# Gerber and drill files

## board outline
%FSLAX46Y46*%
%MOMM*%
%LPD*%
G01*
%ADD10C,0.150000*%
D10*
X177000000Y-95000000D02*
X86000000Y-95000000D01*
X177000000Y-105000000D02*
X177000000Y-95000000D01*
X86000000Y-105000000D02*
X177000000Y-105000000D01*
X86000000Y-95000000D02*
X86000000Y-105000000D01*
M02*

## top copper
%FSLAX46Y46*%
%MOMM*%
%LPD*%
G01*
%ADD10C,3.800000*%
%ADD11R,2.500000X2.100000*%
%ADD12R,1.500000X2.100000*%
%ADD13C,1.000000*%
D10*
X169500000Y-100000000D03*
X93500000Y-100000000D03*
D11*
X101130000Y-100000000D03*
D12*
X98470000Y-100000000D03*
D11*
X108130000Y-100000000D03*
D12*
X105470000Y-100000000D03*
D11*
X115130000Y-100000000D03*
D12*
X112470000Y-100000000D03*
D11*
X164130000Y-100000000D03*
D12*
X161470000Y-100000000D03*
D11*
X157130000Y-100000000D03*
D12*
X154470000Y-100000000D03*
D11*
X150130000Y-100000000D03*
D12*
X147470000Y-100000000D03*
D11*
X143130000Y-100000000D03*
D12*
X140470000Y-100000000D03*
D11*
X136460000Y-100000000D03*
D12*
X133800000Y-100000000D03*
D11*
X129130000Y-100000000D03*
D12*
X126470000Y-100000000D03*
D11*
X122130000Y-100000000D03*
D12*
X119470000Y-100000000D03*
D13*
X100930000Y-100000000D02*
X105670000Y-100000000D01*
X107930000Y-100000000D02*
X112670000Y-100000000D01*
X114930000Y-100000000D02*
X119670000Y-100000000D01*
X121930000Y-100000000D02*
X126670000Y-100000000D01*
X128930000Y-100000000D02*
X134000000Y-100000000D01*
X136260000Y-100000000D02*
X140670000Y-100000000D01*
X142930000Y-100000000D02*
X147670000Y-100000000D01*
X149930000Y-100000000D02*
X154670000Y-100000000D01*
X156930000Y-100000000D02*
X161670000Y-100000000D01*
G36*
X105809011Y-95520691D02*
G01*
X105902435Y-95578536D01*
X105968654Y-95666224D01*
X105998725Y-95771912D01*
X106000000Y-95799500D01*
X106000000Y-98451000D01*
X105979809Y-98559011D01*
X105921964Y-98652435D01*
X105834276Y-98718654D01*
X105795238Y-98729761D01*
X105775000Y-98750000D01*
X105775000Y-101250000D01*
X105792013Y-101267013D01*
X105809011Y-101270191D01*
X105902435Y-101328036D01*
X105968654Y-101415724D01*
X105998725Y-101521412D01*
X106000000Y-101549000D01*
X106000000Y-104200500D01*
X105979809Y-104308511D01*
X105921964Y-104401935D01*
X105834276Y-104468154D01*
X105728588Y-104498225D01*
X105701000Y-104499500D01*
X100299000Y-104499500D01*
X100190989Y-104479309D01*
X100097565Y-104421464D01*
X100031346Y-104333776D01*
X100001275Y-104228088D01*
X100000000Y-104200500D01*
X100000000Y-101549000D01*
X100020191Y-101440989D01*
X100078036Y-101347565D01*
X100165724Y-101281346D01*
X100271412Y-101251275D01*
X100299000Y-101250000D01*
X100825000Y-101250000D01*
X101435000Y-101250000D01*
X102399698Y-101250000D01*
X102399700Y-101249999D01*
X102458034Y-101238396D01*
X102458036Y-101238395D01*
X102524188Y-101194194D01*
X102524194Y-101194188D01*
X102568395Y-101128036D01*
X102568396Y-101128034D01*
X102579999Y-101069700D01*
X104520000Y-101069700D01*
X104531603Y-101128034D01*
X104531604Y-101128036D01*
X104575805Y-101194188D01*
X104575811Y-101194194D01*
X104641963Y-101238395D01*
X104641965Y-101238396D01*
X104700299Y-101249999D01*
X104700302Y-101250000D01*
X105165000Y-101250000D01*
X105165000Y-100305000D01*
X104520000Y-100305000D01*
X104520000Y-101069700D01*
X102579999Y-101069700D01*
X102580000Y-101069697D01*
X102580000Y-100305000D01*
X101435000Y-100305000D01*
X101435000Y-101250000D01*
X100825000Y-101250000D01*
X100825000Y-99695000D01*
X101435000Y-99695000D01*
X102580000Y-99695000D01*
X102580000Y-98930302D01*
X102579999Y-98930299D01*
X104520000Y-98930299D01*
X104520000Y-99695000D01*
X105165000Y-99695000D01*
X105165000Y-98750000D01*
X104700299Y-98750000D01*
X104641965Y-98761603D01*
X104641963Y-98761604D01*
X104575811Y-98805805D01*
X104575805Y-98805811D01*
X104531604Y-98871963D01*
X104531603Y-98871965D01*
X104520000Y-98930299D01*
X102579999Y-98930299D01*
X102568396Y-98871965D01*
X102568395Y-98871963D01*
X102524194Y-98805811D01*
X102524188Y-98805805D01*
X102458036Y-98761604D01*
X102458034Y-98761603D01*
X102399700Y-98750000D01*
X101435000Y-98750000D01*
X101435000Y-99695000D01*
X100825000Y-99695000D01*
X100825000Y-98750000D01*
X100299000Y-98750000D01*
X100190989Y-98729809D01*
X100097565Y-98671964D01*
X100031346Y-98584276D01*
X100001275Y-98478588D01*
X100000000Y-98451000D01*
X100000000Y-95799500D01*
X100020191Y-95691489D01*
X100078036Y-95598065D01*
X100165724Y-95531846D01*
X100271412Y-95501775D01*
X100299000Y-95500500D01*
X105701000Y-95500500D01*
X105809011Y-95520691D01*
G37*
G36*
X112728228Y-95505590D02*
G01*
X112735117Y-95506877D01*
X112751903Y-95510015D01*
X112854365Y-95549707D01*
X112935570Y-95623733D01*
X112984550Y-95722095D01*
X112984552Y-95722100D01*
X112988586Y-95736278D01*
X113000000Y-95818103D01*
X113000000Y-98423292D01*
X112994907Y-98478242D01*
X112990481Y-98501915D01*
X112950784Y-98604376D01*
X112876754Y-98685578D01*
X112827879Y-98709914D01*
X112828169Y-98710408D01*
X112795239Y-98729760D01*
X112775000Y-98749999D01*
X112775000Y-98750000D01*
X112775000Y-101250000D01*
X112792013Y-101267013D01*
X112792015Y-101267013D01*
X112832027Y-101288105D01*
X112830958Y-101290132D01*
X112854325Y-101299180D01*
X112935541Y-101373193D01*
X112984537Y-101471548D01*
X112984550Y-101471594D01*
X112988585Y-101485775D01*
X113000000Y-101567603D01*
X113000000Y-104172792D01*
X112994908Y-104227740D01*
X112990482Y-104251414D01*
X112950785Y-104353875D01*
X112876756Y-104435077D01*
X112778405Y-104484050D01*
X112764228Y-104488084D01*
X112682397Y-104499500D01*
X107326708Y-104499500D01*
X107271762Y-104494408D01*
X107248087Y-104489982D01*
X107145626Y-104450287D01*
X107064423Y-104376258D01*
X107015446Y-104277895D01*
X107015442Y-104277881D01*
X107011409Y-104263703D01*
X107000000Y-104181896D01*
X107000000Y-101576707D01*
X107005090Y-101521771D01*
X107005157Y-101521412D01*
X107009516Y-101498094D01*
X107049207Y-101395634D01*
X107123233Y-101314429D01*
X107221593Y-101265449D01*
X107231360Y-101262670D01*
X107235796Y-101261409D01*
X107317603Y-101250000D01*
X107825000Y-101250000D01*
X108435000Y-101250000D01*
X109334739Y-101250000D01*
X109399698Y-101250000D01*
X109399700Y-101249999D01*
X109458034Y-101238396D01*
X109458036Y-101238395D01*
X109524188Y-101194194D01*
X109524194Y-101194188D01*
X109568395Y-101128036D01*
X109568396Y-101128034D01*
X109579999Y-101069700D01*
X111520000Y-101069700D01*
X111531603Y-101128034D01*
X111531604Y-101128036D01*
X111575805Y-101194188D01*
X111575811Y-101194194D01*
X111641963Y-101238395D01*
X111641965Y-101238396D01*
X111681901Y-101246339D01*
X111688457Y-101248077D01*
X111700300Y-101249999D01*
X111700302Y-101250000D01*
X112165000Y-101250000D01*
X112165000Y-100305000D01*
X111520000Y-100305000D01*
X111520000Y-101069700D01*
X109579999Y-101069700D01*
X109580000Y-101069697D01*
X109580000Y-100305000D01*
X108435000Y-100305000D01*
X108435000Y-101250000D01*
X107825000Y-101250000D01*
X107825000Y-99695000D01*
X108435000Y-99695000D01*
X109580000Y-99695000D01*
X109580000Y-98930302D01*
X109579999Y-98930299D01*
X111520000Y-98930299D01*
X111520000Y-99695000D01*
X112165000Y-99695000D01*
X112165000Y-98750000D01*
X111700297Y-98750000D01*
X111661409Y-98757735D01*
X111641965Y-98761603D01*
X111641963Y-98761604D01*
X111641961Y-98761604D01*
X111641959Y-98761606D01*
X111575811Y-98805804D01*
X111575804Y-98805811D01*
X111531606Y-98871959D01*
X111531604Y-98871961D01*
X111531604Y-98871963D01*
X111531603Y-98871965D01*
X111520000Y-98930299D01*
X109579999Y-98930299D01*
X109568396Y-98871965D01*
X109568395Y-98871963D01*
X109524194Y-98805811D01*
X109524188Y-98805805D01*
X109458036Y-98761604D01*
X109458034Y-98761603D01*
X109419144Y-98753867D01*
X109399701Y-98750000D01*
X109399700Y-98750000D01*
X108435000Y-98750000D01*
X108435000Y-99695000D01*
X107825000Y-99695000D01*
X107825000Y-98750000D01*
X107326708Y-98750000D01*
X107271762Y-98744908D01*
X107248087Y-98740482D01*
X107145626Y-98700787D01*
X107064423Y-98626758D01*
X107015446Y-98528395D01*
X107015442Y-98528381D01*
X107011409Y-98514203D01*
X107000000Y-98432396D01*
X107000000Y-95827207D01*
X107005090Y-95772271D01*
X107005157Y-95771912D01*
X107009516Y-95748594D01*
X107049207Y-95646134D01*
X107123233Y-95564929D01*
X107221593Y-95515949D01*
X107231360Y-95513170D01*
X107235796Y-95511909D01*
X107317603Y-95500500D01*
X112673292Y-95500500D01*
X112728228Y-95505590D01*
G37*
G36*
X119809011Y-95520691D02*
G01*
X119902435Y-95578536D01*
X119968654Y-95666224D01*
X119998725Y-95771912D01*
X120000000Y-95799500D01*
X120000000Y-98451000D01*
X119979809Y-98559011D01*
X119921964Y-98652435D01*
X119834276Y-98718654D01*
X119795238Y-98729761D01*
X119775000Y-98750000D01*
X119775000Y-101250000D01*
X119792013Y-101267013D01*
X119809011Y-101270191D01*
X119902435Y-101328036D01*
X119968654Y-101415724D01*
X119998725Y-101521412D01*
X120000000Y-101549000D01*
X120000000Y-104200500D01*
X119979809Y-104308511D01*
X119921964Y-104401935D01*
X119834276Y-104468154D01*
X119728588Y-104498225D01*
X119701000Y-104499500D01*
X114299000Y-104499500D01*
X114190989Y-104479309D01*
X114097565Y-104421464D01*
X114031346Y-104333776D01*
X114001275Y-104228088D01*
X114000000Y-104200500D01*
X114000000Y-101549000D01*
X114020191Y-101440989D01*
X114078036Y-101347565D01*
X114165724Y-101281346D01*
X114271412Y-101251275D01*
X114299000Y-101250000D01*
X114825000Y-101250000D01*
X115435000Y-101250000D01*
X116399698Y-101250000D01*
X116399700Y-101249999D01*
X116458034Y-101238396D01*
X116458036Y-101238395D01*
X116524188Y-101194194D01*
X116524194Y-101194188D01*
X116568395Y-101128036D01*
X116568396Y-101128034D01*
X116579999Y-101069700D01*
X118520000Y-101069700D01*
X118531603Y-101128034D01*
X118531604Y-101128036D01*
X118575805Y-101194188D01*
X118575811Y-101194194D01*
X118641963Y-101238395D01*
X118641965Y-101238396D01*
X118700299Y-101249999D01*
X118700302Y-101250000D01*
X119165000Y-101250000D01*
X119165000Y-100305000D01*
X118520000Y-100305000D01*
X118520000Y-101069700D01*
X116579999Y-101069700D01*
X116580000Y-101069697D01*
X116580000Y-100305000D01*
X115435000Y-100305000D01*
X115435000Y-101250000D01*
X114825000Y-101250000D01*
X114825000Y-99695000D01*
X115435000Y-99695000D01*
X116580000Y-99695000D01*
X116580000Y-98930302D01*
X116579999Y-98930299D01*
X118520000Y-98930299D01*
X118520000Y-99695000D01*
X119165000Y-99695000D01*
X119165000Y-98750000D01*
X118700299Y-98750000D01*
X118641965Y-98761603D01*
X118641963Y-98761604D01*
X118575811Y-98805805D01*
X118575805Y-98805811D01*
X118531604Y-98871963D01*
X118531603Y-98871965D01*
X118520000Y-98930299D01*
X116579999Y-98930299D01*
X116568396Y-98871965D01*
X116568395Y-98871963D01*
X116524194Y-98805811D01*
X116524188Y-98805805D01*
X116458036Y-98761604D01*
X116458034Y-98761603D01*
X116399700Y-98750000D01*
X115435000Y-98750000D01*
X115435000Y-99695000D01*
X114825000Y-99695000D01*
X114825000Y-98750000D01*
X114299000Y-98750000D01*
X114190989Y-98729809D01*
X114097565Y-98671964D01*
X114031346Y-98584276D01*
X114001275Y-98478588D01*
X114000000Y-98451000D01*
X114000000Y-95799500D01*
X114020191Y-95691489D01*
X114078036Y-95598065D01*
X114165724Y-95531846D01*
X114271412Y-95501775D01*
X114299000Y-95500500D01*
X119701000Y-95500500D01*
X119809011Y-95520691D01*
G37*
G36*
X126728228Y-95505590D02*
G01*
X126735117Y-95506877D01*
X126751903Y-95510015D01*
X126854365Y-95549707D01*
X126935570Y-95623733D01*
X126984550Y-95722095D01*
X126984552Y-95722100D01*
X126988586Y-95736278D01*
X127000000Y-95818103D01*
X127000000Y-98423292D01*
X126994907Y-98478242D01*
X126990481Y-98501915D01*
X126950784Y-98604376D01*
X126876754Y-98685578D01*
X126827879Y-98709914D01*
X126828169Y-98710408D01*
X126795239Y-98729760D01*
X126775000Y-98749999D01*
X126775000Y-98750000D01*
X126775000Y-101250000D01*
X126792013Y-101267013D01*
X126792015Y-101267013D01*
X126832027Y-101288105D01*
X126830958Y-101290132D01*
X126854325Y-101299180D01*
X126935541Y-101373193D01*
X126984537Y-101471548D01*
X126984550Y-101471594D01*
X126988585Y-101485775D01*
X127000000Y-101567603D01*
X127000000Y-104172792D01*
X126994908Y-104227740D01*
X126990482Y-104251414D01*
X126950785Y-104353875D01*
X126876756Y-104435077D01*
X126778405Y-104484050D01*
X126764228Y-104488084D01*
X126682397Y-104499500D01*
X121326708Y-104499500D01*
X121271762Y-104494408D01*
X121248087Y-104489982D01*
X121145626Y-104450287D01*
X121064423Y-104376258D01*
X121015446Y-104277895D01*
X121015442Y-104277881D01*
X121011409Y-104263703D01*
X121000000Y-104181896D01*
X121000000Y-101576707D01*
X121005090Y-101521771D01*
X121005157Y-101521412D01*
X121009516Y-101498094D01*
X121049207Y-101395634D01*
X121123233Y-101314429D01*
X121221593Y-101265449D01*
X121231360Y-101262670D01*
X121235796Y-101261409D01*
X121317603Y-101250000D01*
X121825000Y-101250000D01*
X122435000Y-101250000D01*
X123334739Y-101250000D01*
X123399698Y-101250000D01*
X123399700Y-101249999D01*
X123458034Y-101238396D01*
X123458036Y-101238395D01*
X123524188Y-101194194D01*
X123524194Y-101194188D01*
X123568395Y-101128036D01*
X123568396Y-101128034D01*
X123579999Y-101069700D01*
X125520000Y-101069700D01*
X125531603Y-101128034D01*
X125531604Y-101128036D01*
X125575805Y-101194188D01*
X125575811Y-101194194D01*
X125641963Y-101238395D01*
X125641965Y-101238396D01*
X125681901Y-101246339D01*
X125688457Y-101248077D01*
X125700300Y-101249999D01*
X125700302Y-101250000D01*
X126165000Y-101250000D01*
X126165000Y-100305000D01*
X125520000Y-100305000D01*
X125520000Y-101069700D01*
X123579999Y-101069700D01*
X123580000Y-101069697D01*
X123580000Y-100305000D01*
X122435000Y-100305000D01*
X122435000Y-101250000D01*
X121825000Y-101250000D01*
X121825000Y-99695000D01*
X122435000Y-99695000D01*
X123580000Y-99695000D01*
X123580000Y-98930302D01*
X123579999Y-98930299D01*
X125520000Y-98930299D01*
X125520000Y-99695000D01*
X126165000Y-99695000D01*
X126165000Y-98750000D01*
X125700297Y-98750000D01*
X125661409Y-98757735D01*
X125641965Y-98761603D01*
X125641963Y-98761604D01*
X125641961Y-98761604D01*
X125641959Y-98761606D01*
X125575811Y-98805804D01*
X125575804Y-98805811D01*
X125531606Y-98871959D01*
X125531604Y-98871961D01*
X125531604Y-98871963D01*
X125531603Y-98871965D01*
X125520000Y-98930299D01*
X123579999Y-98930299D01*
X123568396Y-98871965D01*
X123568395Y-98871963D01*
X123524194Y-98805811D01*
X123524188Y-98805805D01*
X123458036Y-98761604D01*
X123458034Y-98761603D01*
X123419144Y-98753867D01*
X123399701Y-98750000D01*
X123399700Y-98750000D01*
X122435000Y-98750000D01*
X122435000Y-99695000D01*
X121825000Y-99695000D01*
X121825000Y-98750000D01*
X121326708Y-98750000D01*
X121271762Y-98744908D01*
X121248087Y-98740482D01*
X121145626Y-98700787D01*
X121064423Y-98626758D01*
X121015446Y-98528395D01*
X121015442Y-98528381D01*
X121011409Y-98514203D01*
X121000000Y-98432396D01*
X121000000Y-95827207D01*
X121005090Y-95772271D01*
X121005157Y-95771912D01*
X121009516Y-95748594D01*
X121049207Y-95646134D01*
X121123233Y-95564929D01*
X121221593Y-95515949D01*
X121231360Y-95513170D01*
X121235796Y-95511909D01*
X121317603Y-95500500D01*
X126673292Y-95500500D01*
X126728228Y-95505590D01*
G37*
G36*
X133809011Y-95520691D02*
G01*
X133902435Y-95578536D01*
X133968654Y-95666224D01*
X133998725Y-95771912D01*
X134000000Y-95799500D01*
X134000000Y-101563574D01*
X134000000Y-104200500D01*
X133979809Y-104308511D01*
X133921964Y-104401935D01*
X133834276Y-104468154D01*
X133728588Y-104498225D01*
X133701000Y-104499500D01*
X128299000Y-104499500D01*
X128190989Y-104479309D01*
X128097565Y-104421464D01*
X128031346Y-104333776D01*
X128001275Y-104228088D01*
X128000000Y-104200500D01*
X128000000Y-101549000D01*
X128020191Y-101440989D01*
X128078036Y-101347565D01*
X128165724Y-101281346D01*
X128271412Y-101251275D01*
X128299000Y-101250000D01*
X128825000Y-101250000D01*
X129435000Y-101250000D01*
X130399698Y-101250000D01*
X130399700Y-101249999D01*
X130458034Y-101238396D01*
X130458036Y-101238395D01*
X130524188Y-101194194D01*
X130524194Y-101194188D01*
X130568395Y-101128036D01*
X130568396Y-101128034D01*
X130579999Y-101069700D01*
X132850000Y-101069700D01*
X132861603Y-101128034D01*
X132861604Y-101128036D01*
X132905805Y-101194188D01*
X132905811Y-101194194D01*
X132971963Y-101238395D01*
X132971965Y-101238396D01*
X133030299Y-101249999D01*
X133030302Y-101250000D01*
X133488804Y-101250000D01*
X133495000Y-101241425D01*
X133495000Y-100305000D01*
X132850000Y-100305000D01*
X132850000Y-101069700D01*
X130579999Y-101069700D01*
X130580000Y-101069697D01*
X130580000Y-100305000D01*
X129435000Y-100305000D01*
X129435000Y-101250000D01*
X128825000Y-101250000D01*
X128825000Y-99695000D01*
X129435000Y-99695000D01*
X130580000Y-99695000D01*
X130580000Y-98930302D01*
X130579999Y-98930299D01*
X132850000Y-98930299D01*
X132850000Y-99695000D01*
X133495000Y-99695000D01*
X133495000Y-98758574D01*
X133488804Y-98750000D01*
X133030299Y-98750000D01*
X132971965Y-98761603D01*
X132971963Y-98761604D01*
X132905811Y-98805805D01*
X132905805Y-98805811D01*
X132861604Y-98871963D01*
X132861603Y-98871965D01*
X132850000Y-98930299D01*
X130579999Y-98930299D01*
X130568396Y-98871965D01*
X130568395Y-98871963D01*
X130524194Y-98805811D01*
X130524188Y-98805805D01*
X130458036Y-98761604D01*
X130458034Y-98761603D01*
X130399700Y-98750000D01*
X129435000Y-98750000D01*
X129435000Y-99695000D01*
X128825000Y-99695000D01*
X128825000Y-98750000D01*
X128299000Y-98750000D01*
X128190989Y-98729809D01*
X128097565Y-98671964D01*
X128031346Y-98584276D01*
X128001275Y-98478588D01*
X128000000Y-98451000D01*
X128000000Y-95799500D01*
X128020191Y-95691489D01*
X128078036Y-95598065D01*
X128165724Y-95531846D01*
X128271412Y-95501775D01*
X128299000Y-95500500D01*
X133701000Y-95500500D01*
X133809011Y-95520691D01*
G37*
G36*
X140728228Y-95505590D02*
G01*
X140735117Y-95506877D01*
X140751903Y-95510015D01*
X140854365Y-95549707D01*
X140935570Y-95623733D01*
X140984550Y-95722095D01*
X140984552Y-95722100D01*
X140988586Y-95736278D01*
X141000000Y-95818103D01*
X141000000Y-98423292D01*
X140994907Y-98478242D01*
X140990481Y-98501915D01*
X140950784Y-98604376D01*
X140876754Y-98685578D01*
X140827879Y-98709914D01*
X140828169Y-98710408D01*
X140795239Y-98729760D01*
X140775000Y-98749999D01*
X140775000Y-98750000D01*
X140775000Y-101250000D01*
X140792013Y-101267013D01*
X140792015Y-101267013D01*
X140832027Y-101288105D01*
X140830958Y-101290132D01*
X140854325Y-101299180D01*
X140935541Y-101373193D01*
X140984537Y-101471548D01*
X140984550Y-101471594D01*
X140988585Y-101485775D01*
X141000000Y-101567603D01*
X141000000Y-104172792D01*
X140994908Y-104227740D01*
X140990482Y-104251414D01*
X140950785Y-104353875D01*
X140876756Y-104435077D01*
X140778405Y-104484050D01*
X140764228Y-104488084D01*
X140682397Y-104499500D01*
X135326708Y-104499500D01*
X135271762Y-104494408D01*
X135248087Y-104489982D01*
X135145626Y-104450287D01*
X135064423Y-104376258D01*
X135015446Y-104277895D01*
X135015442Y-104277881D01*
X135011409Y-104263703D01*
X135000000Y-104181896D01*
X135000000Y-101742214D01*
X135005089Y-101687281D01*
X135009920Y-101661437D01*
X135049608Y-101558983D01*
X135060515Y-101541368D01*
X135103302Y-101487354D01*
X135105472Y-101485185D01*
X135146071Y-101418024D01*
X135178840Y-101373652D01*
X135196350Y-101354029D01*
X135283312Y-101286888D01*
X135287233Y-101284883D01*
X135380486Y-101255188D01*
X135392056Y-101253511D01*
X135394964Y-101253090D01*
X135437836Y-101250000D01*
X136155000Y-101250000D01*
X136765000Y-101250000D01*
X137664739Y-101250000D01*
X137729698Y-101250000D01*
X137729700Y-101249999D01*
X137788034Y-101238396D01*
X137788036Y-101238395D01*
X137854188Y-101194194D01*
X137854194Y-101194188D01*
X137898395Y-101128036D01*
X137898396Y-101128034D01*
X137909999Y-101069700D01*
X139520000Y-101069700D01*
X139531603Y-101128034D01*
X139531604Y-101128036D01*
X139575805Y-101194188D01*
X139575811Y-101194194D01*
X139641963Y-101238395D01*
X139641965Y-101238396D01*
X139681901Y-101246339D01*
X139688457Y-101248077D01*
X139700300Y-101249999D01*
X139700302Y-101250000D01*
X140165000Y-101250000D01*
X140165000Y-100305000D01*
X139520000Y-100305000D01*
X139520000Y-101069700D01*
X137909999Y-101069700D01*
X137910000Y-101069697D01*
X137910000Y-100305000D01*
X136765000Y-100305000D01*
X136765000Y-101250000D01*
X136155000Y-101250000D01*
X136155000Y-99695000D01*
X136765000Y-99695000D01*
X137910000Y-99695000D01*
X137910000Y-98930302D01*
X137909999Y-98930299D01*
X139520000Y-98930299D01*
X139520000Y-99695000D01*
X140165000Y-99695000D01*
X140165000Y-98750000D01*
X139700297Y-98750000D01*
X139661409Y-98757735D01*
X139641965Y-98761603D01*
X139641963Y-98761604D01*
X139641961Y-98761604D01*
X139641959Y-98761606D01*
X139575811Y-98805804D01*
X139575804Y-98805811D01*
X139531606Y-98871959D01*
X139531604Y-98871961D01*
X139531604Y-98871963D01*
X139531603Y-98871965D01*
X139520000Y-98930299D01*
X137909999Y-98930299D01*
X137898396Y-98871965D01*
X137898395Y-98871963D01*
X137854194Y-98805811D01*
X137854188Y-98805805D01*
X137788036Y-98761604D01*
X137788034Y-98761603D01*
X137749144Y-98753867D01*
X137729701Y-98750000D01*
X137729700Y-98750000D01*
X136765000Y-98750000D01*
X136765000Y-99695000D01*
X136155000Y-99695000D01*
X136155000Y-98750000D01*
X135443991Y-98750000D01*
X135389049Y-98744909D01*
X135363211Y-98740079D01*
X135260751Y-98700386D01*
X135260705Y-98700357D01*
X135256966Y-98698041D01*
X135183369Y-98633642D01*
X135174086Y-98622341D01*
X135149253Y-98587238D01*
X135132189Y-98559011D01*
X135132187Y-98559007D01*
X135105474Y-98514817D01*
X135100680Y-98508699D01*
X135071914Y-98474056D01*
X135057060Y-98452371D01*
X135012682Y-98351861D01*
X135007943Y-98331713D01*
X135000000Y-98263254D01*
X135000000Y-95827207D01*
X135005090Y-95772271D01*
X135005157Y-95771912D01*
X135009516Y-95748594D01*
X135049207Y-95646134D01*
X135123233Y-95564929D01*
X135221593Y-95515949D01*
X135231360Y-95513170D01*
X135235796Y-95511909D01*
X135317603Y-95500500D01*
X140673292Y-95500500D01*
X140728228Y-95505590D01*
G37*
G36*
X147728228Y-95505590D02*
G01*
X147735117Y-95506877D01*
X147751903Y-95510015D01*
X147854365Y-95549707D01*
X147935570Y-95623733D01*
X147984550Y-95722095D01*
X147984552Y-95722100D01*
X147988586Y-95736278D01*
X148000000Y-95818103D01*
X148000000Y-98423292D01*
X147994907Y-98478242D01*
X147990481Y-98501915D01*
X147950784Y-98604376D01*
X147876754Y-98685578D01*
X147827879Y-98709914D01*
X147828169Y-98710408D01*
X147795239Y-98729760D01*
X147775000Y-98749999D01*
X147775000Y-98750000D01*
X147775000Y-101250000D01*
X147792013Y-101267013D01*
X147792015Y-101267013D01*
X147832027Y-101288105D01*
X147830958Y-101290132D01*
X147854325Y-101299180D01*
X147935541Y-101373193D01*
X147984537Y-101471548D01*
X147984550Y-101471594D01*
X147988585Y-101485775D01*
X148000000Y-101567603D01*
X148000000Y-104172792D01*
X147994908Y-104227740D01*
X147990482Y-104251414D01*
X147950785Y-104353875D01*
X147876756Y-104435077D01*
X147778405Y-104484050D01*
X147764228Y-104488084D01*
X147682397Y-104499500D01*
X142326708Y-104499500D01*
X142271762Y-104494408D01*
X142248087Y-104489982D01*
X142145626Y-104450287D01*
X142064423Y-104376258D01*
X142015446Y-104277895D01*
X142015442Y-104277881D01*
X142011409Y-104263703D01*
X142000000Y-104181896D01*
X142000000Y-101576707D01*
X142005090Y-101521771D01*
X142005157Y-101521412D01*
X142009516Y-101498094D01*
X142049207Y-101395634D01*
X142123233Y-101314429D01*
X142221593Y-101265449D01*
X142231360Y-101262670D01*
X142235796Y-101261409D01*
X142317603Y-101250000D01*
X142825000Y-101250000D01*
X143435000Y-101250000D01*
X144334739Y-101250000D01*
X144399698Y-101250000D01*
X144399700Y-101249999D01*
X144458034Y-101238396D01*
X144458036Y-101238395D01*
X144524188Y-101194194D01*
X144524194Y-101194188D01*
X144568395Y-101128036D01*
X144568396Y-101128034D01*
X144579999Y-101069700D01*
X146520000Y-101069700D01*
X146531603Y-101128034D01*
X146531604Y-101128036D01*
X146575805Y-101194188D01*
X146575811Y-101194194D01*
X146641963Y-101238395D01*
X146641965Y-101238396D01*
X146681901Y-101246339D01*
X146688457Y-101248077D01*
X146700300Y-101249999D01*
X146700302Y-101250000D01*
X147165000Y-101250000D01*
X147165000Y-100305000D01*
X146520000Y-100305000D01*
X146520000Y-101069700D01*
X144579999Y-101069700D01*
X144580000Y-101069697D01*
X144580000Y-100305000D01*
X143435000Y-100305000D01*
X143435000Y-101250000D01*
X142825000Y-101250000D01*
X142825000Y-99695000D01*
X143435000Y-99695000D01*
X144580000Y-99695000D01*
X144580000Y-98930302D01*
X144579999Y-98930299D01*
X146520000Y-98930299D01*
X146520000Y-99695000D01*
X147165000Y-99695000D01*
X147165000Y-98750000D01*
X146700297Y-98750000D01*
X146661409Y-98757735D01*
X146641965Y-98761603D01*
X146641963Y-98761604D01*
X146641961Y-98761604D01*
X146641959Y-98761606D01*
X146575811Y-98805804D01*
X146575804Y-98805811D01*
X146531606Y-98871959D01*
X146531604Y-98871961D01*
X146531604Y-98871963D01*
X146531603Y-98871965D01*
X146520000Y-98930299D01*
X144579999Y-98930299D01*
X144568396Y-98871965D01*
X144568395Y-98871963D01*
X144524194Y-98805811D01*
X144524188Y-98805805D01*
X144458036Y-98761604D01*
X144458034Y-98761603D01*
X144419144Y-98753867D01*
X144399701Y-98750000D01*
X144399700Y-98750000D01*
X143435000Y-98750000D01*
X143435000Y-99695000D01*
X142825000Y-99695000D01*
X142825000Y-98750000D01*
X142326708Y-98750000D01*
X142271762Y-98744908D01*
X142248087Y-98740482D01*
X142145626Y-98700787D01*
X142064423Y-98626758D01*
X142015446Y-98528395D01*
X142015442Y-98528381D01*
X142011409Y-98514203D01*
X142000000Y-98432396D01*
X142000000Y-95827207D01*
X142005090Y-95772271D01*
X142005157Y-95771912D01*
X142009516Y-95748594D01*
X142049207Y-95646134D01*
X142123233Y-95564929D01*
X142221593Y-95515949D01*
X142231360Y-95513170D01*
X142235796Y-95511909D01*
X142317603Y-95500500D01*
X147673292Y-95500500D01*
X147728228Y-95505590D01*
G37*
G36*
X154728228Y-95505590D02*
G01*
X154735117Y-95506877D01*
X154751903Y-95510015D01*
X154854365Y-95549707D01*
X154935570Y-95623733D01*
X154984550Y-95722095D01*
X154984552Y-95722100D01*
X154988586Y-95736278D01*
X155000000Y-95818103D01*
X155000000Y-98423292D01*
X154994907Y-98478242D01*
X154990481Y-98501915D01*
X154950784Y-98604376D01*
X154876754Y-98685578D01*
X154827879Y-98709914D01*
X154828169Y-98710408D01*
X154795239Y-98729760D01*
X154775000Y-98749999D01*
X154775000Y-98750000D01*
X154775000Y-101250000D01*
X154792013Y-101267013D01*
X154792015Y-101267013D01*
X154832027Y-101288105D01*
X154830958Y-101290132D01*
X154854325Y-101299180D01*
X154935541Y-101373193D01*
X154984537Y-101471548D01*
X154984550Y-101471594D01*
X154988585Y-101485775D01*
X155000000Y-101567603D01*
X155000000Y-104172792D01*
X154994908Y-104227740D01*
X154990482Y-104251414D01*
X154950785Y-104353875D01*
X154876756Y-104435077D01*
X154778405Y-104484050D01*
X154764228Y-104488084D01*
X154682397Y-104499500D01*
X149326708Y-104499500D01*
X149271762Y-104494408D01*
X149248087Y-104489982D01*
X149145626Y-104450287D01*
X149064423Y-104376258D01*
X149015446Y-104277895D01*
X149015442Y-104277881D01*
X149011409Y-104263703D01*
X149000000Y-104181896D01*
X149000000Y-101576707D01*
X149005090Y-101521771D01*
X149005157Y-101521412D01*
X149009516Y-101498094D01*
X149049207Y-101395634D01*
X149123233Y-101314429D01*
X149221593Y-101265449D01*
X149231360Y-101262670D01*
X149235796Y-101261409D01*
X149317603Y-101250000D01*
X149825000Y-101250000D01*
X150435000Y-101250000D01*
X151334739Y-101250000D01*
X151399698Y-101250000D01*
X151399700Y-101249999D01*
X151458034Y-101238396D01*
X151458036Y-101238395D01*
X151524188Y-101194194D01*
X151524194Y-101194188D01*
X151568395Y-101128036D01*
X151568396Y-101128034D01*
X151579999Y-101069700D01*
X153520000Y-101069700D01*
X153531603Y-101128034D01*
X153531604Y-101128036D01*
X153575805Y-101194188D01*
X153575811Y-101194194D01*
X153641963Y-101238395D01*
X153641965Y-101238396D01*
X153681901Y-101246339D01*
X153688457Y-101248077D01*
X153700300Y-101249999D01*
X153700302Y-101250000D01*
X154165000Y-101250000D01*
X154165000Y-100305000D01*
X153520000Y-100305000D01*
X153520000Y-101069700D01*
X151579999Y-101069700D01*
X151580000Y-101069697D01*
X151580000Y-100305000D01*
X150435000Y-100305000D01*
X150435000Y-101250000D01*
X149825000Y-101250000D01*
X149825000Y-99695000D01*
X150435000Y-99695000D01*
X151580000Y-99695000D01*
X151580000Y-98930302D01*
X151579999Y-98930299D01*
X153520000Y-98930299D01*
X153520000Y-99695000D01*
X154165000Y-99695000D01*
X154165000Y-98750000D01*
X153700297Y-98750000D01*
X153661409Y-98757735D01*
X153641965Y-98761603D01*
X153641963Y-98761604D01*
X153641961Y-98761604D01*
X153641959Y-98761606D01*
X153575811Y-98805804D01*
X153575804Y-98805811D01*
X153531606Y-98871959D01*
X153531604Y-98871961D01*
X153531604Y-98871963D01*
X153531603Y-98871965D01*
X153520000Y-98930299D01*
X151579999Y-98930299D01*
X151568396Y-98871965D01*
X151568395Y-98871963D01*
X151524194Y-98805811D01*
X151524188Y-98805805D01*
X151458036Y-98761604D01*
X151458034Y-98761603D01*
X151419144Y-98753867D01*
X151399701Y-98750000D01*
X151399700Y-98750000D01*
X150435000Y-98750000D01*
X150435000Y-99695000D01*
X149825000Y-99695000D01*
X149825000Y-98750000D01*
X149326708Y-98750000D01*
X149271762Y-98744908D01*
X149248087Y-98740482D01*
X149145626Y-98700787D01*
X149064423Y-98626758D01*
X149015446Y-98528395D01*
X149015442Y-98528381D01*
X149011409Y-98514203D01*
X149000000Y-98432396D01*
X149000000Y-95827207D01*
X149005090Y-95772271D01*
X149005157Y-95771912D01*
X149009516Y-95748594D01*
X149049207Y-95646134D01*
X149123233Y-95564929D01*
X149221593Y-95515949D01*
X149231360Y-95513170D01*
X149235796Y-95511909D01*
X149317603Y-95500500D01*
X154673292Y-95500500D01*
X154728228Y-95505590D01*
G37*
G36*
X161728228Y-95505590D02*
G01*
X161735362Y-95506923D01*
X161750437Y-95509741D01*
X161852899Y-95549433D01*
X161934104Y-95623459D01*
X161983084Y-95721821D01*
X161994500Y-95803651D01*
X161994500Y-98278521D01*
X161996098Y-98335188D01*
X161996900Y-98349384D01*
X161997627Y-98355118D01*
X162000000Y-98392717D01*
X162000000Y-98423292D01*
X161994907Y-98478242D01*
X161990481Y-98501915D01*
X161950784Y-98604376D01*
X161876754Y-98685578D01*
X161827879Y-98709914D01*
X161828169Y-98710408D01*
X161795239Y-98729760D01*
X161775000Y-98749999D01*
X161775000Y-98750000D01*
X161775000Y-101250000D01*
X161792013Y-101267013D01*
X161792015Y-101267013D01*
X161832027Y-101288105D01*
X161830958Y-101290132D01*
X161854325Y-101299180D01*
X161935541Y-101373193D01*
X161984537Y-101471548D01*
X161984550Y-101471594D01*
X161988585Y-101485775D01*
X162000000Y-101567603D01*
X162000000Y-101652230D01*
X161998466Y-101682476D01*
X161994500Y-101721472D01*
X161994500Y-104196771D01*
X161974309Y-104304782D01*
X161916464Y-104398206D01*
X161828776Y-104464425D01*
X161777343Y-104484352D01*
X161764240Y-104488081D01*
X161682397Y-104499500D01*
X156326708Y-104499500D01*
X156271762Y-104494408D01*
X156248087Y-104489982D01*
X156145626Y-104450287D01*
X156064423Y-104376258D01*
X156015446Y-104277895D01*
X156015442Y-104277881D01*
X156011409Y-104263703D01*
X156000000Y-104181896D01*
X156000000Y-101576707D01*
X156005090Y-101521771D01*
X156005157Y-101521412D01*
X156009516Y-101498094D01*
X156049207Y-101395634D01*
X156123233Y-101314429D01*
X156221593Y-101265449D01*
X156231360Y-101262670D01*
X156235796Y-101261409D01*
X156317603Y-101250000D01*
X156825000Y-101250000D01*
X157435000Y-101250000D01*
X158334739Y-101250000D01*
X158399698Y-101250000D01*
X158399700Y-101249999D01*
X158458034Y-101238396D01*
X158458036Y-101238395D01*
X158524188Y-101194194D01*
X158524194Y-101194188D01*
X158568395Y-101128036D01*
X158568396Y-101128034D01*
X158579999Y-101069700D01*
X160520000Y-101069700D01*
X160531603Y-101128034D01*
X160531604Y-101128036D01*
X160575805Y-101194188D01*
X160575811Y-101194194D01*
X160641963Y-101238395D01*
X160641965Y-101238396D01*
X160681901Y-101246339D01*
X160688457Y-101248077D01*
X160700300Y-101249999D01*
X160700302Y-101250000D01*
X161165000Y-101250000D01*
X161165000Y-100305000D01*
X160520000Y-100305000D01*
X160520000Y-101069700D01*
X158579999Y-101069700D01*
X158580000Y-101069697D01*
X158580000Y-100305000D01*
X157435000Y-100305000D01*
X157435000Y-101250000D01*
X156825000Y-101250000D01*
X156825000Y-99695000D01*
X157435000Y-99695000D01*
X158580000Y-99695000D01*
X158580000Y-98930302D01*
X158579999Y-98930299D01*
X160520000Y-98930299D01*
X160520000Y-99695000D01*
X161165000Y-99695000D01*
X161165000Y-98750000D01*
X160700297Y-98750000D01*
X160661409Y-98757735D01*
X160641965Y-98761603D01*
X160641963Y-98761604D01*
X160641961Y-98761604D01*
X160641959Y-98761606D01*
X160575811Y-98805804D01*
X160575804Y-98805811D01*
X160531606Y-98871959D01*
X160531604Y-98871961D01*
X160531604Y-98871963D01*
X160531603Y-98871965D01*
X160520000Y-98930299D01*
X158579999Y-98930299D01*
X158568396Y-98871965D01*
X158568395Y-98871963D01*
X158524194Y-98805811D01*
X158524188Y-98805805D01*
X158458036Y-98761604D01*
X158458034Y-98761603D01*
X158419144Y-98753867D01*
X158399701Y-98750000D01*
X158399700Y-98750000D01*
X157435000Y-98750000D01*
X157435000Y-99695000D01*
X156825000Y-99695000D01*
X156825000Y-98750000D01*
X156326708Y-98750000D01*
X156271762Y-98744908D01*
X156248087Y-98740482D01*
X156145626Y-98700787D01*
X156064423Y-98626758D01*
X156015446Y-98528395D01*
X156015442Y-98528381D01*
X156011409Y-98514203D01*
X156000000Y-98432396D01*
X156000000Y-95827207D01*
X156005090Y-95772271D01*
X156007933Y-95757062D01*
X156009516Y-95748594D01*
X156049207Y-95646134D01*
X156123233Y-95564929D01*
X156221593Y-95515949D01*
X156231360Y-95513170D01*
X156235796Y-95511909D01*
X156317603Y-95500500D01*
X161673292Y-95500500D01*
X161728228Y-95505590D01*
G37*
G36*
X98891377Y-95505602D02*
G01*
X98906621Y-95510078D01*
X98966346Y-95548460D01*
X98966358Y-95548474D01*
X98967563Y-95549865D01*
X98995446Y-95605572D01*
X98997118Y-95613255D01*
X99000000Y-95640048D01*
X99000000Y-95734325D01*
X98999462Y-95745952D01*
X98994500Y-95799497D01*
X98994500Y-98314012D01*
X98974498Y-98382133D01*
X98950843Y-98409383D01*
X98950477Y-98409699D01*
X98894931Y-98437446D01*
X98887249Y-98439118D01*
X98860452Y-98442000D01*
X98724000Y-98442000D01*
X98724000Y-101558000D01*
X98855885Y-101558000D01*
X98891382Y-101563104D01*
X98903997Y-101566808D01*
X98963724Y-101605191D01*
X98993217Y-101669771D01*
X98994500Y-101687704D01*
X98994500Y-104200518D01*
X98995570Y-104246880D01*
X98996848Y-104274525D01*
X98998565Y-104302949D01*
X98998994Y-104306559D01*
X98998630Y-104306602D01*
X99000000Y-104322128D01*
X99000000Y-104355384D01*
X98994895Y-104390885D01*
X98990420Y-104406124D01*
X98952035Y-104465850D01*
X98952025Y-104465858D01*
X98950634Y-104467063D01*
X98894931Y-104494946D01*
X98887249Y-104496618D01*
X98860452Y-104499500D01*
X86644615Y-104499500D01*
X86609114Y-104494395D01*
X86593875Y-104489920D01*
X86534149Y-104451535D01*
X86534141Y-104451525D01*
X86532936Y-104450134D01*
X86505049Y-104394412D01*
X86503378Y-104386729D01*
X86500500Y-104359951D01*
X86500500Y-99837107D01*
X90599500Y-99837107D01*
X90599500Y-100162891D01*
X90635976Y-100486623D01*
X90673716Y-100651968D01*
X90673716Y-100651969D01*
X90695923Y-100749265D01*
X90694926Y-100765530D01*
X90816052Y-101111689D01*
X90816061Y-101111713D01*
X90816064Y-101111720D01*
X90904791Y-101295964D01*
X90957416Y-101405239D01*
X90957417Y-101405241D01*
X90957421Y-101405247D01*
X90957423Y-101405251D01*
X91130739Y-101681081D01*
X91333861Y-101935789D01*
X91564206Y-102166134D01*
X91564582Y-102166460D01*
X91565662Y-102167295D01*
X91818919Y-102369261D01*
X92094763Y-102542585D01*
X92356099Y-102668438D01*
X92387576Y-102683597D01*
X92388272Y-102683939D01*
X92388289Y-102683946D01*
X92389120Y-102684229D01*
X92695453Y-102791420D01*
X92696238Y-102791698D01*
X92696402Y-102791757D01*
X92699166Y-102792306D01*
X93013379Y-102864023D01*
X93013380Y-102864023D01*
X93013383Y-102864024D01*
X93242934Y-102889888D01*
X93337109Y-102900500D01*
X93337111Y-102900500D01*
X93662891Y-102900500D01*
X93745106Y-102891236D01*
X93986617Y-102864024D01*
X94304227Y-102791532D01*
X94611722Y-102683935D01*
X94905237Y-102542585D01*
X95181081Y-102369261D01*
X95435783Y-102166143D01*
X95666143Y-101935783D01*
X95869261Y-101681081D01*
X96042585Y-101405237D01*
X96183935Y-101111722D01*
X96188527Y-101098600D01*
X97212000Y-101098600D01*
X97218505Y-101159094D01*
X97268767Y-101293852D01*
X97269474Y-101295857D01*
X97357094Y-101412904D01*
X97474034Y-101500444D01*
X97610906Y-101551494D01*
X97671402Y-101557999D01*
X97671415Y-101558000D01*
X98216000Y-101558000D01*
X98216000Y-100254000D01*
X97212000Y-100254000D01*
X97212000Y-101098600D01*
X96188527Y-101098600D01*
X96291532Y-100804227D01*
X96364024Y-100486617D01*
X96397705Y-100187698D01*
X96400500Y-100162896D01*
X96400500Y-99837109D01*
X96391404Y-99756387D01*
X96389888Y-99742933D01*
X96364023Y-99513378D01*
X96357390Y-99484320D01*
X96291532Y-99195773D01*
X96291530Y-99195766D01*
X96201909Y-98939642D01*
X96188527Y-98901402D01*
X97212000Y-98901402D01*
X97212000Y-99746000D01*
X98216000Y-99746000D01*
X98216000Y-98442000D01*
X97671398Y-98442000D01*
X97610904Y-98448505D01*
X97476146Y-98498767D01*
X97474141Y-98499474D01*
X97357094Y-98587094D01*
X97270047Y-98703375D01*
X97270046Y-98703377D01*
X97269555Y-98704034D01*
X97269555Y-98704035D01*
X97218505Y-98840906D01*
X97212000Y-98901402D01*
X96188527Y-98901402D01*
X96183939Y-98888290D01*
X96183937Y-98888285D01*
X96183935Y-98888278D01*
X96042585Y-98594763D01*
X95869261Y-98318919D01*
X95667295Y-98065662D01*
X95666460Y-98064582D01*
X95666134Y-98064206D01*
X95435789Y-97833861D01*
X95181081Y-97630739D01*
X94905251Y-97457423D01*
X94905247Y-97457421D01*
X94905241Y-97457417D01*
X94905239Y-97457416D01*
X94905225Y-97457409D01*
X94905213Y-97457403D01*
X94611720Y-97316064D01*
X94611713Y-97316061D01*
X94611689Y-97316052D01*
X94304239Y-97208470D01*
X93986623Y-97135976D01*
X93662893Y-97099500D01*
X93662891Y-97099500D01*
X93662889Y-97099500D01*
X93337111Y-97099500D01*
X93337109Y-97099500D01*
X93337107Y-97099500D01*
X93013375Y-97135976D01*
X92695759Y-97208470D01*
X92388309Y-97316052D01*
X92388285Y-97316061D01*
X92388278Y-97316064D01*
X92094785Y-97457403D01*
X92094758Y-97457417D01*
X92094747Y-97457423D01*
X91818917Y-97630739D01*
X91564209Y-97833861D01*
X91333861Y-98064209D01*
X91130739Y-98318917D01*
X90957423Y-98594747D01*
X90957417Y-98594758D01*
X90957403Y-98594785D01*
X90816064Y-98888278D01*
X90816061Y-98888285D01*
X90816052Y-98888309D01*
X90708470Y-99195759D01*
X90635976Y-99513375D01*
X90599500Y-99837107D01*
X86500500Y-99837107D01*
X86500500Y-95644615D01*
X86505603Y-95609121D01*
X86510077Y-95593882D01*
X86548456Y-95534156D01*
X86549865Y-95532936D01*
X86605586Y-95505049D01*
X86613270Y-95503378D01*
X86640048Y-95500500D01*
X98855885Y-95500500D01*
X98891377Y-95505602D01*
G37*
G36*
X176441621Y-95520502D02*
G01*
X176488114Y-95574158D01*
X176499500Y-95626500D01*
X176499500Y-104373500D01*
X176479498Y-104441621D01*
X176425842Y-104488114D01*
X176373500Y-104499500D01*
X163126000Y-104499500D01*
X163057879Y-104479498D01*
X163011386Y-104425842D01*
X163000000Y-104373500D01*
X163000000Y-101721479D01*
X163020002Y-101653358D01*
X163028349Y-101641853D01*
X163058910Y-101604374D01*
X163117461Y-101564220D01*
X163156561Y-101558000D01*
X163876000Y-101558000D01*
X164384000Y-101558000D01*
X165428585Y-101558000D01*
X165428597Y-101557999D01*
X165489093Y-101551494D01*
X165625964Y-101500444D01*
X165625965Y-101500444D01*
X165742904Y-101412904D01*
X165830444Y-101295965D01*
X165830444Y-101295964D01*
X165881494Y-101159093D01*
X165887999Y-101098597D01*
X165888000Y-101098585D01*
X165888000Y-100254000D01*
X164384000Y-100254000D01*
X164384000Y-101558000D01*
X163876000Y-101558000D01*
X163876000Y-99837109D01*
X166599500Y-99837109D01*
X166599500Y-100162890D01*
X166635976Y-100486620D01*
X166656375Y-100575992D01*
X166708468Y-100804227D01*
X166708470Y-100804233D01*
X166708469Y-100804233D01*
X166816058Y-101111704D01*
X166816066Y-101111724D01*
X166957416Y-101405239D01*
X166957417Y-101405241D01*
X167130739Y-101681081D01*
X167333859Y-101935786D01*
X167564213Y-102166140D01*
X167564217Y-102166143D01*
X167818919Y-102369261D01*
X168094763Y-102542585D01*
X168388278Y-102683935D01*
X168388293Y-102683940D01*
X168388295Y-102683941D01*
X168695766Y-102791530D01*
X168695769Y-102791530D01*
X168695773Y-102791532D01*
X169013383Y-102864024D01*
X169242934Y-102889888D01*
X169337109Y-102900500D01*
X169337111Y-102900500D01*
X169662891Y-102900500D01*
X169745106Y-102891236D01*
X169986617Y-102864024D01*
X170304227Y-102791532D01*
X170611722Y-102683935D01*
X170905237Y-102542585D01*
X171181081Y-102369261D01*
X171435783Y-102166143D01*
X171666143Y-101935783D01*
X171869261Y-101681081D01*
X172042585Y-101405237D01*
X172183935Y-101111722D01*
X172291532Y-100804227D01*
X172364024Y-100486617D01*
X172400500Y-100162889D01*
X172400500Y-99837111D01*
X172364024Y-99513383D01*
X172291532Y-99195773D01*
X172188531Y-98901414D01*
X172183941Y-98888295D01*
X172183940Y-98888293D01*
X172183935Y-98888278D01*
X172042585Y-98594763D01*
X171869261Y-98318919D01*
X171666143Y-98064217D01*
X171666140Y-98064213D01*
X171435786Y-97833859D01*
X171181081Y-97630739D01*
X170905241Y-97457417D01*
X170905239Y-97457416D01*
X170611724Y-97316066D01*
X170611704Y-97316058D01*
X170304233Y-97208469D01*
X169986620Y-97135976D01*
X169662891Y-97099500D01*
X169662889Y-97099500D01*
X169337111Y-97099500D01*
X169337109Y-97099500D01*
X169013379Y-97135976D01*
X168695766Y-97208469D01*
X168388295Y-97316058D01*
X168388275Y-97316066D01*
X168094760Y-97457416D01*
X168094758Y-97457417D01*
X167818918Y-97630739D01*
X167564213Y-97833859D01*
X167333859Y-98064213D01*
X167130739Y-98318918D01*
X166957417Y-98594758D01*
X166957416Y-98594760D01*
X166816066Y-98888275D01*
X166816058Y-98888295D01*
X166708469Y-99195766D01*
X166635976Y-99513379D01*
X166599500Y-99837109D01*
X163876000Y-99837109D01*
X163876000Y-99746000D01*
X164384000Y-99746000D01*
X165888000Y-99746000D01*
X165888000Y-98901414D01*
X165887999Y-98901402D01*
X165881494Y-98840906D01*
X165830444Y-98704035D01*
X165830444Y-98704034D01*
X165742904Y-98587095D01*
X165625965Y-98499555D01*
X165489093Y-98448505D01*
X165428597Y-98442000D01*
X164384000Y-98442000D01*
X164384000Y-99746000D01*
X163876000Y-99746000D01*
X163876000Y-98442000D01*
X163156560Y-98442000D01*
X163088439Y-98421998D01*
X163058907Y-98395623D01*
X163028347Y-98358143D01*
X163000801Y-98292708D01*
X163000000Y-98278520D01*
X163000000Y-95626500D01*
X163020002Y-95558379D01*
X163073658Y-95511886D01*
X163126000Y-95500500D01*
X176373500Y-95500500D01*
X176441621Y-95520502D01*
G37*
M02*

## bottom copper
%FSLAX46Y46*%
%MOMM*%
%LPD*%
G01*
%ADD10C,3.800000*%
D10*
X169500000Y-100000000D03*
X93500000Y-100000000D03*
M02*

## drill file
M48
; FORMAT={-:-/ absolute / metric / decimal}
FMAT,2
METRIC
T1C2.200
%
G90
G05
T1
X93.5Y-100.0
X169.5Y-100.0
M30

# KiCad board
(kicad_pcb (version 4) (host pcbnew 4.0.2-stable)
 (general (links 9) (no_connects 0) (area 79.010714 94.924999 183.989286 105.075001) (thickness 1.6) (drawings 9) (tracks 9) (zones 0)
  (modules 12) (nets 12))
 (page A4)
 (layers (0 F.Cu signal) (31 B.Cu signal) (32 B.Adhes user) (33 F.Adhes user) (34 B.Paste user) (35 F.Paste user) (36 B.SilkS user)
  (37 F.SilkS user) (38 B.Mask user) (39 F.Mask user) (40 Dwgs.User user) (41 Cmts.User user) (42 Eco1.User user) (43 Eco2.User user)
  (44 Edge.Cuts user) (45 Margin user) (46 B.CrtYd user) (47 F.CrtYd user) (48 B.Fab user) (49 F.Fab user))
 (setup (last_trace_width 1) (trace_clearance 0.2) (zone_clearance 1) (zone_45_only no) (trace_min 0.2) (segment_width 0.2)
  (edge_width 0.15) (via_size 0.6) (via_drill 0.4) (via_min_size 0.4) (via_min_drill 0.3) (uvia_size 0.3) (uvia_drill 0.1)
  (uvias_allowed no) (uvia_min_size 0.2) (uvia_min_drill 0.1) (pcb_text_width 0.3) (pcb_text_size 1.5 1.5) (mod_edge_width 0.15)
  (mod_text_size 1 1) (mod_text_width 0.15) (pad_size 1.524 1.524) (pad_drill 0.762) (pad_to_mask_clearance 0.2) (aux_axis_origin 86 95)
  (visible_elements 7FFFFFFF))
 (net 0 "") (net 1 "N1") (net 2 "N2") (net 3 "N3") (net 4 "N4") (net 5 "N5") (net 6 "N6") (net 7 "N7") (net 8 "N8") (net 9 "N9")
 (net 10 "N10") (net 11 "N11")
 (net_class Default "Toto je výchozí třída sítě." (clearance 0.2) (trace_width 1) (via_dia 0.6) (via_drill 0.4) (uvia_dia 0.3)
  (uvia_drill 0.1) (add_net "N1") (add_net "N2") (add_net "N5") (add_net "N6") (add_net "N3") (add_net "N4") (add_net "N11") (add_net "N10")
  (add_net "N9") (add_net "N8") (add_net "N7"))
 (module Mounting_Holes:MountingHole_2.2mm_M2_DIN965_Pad (layer F.Cu) (at 169.5 100)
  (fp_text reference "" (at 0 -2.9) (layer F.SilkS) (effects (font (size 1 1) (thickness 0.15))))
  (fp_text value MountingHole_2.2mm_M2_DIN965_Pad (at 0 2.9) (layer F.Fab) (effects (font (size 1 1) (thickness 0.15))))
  (pad 1 thru_hole circle (at 0 0) (size 3.8 3.8) (drill 2.2) (layers *.Cu *.Mask F.SilkS)))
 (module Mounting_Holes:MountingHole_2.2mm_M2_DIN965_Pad (layer F.Cu) (at 93.5 100)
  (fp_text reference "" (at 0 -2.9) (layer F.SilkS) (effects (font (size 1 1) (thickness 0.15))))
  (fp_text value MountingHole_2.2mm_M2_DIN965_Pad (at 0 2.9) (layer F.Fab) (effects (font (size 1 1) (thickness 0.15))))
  (pad 1 thru_hole circle (at 0 0) (size 3.8 3.8) (drill 2.2) (layers *.Cu *.Mask F.SilkS)))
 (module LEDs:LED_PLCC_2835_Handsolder (layer F.Cu) (at 100 100)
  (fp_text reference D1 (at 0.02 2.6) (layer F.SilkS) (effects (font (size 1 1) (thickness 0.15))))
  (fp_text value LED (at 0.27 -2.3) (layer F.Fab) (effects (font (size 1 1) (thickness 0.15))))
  (pad 1 smd rect (at 1.13 0) (size 2.5 2.1) (layers F.Cu F.Paste F.Mask) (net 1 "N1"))
  (pad 2 smd rect (at -1.53 0) (size 1.5 2.1) (layers F.Cu F.Paste F.Mask) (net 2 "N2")))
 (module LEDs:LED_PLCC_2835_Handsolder (layer F.Cu) (at 107 100)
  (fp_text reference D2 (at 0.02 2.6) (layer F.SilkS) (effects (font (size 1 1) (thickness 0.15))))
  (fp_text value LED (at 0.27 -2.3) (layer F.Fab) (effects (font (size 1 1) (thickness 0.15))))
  (pad 1 smd rect (at 1.13 0) (size 2.5 2.1) (layers F.Cu F.Paste F.Mask) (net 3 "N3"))
  (pad 2 smd rect (at -1.53 0) (size 1.5 2.1) (layers F.Cu F.Paste F.Mask) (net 1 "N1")))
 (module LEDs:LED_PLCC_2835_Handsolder (layer F.Cu) (at 114 100)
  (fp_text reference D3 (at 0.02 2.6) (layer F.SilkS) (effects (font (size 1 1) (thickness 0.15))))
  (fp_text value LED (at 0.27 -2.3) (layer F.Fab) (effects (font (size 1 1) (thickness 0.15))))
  (pad 1 smd rect (at 1.13 0) (size 2.5 2.1) (layers F.Cu F.Paste F.Mask) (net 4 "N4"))
  (pad 2 smd rect (at -1.53 0) (size 1.5 2.1) (layers F.Cu F.Paste F.Mask) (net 3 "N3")))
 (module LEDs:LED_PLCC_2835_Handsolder (layer F.Cu) (at 163 100)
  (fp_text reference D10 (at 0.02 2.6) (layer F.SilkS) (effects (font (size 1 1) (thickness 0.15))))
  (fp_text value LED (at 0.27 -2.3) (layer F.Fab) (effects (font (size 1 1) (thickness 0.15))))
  (pad 1 smd rect (at 1.13 0) (size 2.5 2.1) (layers F.Cu F.Paste F.Mask) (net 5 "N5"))
  (pad 2 smd rect (at -1.53 0) (size 1.5 2.1) (layers F.Cu F.Paste F.Mask) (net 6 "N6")))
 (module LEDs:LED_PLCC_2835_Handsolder (layer F.Cu) (at 156 100)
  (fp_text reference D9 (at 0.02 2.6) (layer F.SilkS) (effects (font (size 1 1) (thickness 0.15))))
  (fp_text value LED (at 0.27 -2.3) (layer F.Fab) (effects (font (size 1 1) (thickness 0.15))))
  (pad 1 smd rect (at 1.13 0) (size 2.5 2.1) (layers F.Cu F.Paste F.Mask) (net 6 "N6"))
  (pad 2 smd rect (at -1.53 0) (size 1.5 2.1) (layers F.Cu F.Paste F.Mask) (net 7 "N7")))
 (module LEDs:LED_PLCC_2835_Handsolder (layer F.Cu) (at 149 100)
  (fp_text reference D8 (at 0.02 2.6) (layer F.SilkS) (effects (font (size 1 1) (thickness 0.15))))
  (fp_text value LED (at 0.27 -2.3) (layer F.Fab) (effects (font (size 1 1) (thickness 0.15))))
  (pad 1 smd rect (at 1.13 0) (size 2.5 2.1) (layers F.Cu F.Paste F.Mask) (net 7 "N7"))
  (pad 2 smd rect (at -1.53 0) (size 1.5 2.1) (layers F.Cu F.Paste F.Mask) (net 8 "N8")))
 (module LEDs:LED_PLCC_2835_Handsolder (layer F.Cu) (at 142 100)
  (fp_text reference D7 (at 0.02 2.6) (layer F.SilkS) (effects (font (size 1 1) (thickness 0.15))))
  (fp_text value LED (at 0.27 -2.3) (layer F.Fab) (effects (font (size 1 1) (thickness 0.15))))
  (pad 1 smd rect (at 1.13 0) (size 2.5 2.1) (layers F.Cu F.Paste F.Mask) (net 8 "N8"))
  (pad 2 smd rect (at -1.53 0) (size 1.5 2.1) (layers F.Cu F.Paste F.Mask) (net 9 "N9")))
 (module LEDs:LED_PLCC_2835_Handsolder (layer F.Cu) (at 135.33 100)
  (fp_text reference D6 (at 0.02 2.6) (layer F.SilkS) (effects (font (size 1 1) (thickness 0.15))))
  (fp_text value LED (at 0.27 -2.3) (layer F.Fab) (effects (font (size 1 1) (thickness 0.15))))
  (pad 1 smd rect (at 1.13 0) (size 2.5 2.1) (layers F.Cu F.Paste F.Mask) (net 9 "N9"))
  (pad 2 smd rect (at -1.53 0) (size 1.5 2.1) (layers F.Cu F.Paste F.Mask) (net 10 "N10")))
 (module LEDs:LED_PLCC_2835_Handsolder (layer F.Cu) (at 128 100)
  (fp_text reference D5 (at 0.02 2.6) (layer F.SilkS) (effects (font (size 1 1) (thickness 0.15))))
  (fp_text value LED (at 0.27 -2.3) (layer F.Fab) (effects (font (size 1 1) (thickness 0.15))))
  (pad 1 smd rect (at 1.13 0) (size 2.5 2.1) (layers F.Cu F.Paste F.Mask) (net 10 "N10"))
  (pad 2 smd rect (at -1.53 0) (size 1.5 2.1) (layers F.Cu F.Paste F.Mask) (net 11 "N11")))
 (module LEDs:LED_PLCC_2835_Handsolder (layer F.Cu) (at 121 100)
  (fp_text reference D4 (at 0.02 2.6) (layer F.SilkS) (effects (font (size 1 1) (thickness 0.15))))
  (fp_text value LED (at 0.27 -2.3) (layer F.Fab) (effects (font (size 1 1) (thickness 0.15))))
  (pad 1 smd rect (at 1.13 0) (size 2.5 2.1) (layers F.Cu F.Paste F.Mask) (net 11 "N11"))
  (pad 2 smd rect (at -1.53 0) (size 1.5 2.1) (layers F.Cu F.Paste F.Mask) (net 4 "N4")))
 (gr_line (start 177 95) (end 86 95) (layer Edge.Cuts) (width 0.15))
 (gr_line (start 177 105) (end 177 95) (layer Edge.Cuts) (width 0.15))
 (gr_line (start 86 105) (end 177 105) (layer Edge.Cuts) (width 0.15))
 (gr_line (start 86 95) (end 86 105) (layer Edge.Cuts) (width 0.15))
 (segment (start 100.93 100) (end 105.67 100) (width 1) (layer F.Cu) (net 1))
 (segment (start 107.93 100) (end 112.67 100) (width 1) (layer F.Cu) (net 3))
 (segment (start 114.93 100) (end 119.67 100) (width 1) (layer F.Cu) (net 4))
 (segment (start 121.93 100) (end 126.67 100) (width 1) (layer F.Cu) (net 11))
 (segment (start 128.93 100) (end 134 100) (width 1) (layer F.Cu) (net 10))
 (segment (start 136.26 100) (end 140.67 100) (width 1) (layer F.Cu) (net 9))
 (segment (start 142.93 100) (end 147.67 100) (width 1) (layer F.Cu) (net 8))
 (segment (start 149.93 100) (end 154.67 100) (width 1) (layer F.Cu) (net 7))
 (segment (start 156.93 100) (end 161.67 100) (width 1) (layer F.Cu) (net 6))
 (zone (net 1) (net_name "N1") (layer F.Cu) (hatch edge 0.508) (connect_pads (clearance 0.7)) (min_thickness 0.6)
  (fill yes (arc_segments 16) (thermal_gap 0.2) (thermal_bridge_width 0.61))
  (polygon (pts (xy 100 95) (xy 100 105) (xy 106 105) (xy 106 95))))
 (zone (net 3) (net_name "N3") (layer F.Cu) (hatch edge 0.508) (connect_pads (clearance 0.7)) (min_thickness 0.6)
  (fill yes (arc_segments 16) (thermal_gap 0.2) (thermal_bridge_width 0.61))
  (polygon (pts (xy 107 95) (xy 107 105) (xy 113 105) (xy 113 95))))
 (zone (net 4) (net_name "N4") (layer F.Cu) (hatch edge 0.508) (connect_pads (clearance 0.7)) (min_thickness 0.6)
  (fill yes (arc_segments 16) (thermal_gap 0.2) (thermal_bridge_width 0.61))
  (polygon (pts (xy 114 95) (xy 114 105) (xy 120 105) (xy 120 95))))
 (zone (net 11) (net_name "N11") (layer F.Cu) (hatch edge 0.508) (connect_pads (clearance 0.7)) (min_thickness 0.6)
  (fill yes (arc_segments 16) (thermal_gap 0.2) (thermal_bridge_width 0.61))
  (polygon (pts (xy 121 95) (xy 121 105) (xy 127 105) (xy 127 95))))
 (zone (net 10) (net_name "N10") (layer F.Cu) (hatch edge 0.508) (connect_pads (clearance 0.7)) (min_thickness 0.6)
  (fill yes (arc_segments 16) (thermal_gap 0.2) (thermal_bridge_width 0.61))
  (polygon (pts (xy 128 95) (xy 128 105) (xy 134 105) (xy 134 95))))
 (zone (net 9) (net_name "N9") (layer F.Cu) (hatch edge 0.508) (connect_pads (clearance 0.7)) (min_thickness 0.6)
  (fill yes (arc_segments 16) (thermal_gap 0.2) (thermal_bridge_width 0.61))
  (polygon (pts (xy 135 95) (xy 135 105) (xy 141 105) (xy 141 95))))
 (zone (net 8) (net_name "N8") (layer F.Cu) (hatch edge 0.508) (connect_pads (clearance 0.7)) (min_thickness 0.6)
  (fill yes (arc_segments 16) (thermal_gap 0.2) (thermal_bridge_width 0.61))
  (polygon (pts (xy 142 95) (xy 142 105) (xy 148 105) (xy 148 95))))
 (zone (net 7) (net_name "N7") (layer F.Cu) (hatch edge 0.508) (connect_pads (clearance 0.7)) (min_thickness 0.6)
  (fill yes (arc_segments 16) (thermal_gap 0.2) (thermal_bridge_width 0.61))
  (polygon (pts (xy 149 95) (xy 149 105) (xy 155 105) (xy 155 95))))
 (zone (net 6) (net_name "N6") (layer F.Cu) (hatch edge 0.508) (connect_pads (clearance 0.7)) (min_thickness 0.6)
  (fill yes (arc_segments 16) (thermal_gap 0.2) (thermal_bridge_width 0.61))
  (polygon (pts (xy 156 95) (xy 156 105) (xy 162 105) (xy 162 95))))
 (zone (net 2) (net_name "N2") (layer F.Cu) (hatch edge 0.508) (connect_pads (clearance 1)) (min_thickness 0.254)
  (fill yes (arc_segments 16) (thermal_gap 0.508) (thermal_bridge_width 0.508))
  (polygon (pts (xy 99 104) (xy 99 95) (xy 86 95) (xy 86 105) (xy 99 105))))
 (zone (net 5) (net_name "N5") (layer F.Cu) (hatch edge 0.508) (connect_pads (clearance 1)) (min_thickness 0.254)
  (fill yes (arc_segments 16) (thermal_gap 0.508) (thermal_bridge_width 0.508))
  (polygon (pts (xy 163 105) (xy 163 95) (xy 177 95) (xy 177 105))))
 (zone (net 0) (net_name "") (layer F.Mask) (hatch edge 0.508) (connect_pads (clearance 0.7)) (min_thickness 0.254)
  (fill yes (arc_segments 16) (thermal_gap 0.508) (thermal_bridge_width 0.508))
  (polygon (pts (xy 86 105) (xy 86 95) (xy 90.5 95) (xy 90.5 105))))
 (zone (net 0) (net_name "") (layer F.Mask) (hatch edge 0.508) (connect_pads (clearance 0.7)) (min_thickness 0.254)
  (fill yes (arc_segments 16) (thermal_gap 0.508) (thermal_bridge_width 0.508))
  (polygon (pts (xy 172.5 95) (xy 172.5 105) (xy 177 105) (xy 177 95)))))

